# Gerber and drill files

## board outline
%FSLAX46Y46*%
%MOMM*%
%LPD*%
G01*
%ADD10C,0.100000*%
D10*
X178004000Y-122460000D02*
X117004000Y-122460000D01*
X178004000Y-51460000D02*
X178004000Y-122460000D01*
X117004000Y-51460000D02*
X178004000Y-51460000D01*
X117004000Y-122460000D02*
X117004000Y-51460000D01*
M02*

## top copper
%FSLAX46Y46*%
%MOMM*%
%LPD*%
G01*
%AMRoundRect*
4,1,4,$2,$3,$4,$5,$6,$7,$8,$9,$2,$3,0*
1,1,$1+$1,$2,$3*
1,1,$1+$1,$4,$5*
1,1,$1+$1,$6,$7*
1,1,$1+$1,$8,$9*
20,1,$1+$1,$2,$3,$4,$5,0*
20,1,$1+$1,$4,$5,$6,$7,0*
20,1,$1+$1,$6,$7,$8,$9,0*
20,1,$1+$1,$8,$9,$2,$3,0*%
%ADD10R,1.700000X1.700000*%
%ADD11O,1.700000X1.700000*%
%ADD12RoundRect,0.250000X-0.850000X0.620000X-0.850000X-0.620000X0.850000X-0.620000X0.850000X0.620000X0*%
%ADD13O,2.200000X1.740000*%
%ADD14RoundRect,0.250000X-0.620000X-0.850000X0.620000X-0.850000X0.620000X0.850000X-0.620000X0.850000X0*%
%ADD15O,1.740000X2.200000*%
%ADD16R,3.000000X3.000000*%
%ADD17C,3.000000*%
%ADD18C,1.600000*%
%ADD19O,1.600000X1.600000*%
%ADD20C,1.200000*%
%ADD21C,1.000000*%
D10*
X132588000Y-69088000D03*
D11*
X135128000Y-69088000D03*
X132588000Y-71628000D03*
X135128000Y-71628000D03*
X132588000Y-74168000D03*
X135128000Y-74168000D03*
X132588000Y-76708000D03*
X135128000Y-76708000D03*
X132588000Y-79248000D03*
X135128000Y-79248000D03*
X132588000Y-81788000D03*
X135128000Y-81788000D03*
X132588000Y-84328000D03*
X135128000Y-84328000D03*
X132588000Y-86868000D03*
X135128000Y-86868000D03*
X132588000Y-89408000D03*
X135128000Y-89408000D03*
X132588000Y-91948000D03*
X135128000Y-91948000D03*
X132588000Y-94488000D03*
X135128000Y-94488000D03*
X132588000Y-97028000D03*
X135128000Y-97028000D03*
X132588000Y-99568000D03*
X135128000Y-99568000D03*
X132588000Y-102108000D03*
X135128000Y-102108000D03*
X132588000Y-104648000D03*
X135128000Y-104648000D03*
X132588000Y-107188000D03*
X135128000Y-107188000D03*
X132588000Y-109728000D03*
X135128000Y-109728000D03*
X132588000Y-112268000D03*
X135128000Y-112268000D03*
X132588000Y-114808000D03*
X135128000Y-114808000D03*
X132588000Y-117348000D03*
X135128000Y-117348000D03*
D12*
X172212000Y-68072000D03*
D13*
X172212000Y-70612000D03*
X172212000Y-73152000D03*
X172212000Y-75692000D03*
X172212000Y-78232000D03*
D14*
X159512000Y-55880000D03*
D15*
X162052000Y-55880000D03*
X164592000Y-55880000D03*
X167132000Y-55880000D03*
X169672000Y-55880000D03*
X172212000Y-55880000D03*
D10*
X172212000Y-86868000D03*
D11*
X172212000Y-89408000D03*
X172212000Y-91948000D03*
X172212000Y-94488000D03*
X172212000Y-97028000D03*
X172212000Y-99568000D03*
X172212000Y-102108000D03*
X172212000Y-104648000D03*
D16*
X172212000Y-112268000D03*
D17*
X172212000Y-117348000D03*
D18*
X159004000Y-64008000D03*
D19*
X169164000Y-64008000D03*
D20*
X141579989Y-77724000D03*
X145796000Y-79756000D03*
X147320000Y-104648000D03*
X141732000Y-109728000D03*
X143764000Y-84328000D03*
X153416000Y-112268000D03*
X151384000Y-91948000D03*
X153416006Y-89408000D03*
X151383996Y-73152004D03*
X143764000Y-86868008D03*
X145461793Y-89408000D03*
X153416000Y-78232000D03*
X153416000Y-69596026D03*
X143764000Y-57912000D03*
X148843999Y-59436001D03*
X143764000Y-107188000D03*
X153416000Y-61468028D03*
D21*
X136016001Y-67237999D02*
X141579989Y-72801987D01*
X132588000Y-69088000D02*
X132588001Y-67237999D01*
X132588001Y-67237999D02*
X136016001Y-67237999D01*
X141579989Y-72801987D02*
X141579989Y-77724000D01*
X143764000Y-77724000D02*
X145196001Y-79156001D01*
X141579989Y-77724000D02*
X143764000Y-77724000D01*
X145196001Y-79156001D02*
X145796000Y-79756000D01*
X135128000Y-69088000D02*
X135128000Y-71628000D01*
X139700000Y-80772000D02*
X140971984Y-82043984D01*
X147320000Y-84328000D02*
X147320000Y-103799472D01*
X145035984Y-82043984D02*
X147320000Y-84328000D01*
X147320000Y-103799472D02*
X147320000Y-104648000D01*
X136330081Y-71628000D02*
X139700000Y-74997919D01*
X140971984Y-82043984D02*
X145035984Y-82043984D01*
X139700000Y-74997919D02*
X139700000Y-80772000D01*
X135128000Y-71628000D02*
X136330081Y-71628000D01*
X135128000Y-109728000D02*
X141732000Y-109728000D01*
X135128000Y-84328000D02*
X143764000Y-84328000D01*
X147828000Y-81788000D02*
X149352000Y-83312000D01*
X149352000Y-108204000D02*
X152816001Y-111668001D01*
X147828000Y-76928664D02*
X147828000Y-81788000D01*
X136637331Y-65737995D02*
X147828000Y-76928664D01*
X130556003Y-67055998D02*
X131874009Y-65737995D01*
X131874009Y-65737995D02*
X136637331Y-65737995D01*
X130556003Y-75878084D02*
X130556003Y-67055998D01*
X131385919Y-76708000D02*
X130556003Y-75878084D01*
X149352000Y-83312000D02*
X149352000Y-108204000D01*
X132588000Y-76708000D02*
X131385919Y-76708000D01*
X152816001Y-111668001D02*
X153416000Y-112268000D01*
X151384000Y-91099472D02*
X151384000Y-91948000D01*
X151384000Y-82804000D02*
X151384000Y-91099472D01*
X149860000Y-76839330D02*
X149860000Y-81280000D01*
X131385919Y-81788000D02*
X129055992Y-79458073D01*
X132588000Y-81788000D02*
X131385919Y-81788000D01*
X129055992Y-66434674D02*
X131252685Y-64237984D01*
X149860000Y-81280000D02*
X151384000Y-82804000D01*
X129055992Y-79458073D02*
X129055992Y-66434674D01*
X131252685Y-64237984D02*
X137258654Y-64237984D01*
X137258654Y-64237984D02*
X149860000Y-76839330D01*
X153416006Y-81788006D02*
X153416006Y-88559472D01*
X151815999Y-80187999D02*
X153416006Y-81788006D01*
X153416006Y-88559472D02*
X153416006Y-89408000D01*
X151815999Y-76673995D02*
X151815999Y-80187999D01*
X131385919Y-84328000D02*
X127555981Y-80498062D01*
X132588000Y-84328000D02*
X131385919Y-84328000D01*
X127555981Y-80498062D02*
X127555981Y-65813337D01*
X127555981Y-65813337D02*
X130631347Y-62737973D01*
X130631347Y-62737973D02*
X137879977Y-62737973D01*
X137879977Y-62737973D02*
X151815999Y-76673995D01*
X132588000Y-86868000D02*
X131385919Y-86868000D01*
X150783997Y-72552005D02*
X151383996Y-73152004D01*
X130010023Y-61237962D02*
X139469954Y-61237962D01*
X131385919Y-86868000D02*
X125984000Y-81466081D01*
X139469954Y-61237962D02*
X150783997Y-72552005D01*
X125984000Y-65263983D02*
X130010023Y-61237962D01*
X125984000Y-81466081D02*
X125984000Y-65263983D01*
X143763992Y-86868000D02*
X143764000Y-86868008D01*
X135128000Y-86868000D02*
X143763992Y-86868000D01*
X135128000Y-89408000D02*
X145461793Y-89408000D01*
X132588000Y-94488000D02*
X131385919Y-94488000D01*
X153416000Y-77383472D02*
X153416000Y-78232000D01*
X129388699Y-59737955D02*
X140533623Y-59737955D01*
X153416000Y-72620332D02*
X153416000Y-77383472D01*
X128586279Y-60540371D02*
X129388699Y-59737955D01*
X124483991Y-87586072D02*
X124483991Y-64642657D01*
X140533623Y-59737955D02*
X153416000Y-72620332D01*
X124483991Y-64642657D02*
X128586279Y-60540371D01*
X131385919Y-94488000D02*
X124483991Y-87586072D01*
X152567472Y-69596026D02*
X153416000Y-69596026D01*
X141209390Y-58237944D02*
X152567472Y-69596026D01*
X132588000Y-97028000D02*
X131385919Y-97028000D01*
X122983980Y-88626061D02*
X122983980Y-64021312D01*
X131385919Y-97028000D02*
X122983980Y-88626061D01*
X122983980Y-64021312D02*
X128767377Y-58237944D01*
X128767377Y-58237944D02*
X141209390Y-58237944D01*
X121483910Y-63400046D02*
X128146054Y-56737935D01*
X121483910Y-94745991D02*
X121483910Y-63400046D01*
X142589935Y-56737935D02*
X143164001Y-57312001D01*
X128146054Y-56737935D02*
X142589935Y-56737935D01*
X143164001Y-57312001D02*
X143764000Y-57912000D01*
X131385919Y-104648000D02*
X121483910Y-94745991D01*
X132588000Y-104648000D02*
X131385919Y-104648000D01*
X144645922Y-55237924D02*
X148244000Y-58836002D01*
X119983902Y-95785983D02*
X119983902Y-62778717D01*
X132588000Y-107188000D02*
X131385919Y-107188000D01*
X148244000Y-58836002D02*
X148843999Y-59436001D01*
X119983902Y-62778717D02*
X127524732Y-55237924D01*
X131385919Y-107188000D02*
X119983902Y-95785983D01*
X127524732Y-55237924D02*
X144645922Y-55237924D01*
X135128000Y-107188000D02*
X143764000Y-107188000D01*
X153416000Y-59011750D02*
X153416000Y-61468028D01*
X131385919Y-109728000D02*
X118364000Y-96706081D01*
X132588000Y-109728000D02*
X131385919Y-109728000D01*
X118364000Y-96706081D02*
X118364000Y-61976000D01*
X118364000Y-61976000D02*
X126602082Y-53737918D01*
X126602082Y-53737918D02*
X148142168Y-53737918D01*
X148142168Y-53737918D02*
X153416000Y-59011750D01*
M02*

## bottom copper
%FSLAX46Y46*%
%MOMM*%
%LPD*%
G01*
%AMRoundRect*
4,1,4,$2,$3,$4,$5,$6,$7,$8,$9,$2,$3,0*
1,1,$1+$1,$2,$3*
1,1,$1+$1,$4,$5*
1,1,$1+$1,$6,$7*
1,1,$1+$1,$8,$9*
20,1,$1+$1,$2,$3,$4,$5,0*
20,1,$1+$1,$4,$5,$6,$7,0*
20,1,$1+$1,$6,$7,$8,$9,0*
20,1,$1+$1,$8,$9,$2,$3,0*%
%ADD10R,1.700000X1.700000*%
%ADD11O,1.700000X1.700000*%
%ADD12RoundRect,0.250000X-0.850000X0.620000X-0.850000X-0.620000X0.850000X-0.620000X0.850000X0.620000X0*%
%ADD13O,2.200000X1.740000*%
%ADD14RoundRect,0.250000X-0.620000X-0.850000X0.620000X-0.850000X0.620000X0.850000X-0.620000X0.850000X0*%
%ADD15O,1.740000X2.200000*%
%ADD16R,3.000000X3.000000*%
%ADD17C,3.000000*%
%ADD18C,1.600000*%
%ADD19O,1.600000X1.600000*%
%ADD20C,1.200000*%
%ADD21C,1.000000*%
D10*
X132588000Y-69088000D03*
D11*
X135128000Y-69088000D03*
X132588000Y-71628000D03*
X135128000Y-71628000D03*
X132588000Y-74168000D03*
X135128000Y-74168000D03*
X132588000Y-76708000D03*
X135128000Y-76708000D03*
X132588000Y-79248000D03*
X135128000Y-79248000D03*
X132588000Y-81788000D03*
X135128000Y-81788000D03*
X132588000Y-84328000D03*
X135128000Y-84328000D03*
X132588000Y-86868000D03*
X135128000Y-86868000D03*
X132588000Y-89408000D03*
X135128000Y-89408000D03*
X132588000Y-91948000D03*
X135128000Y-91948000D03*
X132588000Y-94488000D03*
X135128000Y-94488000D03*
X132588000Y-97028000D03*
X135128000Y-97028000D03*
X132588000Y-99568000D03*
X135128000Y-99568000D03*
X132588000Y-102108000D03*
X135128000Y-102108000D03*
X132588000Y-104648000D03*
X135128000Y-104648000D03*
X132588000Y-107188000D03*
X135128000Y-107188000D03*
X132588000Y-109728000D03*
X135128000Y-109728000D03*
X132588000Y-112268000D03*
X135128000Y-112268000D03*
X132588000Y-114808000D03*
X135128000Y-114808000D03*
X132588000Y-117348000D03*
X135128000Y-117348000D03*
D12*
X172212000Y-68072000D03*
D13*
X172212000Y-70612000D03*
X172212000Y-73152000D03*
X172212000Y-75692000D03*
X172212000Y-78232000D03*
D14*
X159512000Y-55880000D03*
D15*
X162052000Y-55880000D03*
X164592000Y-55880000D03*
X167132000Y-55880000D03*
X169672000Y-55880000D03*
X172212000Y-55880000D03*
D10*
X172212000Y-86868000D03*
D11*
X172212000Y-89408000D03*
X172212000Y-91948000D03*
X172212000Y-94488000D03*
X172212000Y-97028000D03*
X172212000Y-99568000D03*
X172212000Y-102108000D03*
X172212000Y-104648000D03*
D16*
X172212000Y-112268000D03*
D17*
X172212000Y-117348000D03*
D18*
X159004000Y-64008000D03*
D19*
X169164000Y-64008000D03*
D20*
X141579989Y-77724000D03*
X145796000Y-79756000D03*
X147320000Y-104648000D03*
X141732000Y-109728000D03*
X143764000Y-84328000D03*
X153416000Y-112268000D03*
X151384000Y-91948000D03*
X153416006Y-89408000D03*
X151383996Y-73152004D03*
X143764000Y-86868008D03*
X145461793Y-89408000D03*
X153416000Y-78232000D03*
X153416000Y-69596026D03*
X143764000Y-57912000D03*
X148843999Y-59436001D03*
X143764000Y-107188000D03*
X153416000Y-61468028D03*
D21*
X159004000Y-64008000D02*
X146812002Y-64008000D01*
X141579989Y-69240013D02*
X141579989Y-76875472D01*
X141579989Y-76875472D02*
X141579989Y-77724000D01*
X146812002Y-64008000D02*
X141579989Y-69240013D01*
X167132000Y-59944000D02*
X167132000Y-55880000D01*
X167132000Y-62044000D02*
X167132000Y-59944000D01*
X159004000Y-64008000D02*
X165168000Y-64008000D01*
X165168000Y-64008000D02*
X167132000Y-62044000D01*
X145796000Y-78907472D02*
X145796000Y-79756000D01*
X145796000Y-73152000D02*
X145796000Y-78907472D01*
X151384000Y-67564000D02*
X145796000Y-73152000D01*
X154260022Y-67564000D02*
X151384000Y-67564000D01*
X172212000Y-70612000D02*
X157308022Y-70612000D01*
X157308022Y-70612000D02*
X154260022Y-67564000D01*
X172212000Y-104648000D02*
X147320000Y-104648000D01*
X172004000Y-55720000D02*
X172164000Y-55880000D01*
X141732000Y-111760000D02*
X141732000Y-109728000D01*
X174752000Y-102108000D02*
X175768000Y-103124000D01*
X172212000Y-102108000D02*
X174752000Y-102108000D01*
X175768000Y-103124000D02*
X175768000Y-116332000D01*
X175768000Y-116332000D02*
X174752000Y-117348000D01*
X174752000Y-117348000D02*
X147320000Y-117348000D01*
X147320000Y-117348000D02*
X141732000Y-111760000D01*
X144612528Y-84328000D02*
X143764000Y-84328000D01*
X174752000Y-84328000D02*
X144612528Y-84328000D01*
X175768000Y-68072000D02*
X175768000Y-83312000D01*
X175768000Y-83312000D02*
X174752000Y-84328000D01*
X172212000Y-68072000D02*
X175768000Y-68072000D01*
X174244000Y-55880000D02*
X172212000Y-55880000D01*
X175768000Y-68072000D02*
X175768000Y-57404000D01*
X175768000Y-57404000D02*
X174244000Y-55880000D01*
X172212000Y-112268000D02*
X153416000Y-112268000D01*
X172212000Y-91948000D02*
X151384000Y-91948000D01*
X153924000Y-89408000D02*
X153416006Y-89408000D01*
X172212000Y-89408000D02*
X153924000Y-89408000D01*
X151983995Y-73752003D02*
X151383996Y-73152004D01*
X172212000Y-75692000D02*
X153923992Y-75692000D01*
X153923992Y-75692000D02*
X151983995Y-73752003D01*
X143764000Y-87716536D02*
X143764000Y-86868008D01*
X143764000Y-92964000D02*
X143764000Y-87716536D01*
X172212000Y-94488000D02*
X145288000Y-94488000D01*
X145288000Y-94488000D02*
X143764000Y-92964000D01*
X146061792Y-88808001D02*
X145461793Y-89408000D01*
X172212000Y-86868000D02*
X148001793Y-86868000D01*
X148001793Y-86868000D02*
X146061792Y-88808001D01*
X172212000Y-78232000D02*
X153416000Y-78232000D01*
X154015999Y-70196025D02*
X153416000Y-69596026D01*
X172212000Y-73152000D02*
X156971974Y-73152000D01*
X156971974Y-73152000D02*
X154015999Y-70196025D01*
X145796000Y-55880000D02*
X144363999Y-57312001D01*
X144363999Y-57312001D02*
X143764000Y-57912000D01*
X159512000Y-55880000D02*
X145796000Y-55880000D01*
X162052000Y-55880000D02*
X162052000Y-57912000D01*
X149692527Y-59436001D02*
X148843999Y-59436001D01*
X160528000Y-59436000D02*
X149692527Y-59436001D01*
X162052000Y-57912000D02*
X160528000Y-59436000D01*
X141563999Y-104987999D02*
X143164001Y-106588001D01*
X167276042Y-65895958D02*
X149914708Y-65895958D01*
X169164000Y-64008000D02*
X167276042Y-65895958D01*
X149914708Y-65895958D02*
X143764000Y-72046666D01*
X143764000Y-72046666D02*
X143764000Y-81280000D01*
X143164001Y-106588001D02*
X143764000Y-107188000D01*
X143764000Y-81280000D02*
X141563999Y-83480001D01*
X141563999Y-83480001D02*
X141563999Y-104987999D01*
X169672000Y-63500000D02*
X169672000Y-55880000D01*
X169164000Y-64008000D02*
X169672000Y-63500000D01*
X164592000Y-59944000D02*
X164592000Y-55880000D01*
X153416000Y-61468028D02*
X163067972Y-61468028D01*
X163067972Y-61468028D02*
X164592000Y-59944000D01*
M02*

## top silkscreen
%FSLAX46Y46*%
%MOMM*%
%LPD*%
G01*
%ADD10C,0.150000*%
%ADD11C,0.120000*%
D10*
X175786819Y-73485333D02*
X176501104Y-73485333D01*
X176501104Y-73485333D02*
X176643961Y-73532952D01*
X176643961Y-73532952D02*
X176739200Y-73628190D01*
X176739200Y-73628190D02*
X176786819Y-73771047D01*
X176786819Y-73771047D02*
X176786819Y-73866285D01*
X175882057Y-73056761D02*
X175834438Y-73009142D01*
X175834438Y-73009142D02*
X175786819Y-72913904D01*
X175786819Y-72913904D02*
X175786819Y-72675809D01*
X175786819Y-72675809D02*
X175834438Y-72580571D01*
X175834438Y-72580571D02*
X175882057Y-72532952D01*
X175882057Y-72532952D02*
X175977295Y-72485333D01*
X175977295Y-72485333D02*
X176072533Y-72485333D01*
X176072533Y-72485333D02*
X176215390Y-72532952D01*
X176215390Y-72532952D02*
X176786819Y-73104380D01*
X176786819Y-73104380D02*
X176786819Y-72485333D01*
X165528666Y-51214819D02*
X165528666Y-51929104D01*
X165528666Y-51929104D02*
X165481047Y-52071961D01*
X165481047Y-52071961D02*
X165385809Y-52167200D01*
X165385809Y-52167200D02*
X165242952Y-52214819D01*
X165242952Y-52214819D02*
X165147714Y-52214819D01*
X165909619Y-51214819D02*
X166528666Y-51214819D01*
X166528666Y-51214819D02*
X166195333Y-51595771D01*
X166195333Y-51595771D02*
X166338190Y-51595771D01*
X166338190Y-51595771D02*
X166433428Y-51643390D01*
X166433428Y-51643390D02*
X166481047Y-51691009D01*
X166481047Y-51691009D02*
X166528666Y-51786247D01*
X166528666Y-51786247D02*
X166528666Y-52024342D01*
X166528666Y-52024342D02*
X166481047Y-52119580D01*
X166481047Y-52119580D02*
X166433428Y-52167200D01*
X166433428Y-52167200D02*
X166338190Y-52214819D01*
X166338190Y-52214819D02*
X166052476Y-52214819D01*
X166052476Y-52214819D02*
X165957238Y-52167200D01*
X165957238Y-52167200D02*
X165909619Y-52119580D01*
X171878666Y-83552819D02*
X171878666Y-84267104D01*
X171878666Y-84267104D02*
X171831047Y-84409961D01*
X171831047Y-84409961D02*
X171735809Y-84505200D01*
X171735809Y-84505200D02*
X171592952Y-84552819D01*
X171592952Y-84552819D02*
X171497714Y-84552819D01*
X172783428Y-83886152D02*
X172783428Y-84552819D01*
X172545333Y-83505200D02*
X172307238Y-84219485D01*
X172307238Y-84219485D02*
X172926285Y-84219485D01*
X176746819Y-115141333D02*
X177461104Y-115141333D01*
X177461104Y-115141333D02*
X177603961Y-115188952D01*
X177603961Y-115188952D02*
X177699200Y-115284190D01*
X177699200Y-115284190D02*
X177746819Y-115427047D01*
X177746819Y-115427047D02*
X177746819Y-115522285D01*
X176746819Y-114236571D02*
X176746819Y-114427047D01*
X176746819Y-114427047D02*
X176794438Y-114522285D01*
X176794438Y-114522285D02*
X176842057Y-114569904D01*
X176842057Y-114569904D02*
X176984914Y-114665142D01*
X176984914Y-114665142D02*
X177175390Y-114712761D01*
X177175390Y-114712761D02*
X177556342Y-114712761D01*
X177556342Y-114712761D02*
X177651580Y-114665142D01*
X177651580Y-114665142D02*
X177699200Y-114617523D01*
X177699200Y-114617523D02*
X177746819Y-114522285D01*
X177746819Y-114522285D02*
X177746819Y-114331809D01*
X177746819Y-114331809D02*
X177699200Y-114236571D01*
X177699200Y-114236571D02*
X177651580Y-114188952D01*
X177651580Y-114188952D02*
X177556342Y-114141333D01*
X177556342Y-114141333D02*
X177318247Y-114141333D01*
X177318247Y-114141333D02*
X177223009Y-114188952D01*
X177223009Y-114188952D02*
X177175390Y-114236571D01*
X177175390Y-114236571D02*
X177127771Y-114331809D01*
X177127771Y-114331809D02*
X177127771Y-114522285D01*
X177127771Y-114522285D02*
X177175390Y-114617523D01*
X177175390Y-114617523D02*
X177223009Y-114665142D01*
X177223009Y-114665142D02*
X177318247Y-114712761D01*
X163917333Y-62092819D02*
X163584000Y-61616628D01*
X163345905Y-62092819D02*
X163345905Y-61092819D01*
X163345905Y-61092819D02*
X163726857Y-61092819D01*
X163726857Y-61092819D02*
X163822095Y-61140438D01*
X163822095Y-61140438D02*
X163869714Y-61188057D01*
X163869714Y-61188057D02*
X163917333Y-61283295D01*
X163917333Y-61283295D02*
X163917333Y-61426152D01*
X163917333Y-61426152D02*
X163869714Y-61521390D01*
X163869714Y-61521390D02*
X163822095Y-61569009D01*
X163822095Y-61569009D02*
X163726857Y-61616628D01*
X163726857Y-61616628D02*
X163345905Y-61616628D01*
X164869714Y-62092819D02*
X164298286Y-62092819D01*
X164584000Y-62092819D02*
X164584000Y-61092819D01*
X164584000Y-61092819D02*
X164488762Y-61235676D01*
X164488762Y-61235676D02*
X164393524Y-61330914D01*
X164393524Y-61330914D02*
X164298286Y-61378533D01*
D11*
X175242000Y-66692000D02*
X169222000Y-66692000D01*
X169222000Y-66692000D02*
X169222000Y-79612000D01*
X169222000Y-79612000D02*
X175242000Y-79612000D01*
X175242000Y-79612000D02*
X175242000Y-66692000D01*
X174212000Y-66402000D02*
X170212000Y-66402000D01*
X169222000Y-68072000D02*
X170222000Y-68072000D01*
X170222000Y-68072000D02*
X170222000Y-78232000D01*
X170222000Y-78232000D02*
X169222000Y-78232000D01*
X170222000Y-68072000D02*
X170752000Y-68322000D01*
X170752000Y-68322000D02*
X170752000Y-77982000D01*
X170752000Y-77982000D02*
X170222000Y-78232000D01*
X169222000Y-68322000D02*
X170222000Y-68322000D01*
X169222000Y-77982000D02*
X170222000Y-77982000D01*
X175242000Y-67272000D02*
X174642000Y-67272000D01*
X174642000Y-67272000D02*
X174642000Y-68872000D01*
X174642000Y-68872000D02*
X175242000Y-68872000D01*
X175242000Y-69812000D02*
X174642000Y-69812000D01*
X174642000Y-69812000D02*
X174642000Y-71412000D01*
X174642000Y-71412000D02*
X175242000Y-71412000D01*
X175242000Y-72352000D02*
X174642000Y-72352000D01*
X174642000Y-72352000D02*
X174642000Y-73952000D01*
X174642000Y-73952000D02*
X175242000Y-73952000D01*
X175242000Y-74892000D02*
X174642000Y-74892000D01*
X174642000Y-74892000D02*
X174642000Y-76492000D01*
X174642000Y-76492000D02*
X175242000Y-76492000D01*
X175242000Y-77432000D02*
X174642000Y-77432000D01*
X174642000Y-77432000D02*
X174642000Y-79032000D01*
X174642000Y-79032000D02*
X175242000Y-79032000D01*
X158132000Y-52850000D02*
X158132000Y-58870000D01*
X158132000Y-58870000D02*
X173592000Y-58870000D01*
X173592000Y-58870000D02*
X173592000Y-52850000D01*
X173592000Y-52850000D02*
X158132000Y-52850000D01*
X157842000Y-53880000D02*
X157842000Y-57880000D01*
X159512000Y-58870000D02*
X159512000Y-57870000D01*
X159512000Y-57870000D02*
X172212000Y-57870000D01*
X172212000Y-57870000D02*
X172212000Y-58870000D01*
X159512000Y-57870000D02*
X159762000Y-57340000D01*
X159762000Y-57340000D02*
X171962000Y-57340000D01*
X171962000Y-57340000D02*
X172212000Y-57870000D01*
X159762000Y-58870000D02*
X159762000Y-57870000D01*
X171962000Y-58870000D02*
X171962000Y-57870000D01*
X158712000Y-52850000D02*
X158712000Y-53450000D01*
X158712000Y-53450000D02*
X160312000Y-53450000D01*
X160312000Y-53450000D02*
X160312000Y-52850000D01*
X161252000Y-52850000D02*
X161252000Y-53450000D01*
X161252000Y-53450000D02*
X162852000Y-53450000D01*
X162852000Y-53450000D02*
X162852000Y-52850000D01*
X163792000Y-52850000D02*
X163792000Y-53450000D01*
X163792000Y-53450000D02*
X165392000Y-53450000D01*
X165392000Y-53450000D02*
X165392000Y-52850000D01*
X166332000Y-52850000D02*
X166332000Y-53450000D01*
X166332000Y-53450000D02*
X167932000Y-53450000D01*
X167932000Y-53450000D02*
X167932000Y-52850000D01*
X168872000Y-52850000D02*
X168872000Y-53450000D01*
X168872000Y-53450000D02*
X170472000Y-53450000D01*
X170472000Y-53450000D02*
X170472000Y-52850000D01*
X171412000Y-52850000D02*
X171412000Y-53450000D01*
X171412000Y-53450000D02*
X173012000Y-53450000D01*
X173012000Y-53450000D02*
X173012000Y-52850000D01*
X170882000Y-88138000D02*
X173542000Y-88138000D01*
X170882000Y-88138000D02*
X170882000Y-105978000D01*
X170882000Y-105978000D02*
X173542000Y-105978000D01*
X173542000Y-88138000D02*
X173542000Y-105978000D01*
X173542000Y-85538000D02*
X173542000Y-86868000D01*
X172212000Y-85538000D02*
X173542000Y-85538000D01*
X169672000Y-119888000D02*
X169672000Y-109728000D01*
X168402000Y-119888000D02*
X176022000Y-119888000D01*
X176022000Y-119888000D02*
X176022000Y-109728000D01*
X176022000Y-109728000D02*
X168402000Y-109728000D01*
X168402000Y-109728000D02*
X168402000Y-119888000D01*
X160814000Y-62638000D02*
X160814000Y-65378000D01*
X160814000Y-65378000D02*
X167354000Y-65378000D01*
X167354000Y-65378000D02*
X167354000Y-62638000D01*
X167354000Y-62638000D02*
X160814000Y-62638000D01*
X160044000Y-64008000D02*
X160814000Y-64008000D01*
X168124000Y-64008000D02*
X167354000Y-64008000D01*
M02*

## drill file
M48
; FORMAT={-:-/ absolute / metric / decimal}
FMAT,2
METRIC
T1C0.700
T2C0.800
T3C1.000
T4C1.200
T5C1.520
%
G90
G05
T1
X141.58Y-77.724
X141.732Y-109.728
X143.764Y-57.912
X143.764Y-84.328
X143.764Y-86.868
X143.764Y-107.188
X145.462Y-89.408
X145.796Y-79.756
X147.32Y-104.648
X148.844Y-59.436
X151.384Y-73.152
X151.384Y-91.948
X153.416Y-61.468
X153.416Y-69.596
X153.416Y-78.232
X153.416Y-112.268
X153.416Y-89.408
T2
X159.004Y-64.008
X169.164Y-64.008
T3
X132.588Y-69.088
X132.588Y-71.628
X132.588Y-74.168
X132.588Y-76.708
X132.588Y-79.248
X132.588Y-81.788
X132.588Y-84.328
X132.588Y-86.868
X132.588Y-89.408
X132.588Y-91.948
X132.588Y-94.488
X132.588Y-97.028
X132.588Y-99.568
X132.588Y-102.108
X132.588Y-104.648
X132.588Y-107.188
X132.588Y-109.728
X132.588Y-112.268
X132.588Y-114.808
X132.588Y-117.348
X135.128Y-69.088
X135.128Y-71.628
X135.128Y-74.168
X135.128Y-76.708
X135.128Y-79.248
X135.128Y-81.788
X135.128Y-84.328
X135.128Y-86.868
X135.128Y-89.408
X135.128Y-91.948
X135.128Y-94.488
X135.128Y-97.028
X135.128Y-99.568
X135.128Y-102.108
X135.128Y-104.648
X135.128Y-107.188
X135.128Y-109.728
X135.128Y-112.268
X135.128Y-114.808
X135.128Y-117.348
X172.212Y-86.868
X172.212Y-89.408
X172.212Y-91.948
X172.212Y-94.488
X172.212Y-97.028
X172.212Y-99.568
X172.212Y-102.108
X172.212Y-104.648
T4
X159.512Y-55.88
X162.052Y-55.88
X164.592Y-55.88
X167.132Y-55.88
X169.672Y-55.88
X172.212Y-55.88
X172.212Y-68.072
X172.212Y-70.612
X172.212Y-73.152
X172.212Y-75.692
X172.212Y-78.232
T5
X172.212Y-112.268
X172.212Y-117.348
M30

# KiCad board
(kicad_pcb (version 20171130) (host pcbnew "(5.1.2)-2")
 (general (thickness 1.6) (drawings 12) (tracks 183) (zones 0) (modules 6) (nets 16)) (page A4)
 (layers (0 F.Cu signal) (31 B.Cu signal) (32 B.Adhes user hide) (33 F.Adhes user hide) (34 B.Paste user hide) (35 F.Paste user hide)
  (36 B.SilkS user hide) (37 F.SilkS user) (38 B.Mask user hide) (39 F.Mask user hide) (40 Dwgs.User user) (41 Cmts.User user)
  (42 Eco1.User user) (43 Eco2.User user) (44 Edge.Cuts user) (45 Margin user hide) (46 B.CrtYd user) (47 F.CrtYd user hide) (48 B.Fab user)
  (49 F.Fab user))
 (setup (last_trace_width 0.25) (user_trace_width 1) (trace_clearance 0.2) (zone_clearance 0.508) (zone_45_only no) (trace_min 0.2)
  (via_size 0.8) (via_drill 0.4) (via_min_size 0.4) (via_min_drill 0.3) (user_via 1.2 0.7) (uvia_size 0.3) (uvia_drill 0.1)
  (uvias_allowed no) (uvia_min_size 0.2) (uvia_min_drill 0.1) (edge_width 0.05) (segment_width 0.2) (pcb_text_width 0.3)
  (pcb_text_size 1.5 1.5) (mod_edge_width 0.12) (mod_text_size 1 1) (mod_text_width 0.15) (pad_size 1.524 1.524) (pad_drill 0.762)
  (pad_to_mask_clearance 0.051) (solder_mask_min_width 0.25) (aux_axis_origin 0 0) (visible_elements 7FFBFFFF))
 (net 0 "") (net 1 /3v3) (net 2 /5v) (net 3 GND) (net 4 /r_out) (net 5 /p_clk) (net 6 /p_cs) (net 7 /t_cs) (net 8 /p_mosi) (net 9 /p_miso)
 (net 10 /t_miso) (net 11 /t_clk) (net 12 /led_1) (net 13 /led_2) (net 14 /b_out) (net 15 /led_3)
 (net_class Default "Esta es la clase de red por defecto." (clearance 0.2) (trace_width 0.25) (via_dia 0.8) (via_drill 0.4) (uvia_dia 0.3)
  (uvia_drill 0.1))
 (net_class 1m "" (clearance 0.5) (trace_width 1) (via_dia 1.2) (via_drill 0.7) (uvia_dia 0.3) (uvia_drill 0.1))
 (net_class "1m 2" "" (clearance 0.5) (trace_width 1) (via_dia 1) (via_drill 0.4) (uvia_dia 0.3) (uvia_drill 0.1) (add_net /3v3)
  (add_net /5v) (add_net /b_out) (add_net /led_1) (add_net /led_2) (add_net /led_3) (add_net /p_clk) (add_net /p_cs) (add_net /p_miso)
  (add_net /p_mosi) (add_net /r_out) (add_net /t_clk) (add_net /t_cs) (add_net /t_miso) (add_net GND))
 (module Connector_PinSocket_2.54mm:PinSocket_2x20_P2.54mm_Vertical (layer B.Cu) (at 132.588 69.088 180)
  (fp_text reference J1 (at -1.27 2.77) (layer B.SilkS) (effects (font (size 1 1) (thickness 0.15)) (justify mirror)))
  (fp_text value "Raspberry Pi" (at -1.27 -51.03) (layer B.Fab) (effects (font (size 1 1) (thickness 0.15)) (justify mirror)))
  (pad 1 thru_hole rect (at 0 0 180) (size 1.7 1.7) (drill 1) (layers *.Cu *.Mask) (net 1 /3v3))
  (pad 2 thru_hole oval (at -2.54 0 180) (size 1.7 1.7) (drill 1) (layers *.Cu *.Mask) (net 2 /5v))
  (pad 3 thru_hole oval (at 0 -2.54 180) (size 1.7 1.7) (drill 1) (layers *.Cu *.Mask))
  (pad 4 thru_hole oval (at -2.54 -2.54 180) (size 1.7 1.7) (drill 1) (layers *.Cu *.Mask) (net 2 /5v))
  (pad 5 thru_hole oval (at 0 -5.08 180) (size 1.7 1.7) (drill 1) (layers *.Cu *.Mask))
  (pad 6 thru_hole oval (at -2.54 -5.08 180) (size 1.7 1.7) (drill 1) (layers *.Cu *.Mask) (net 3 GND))
  (pad 7 thru_hole oval (at 0 -7.62 180) (size 1.7 1.7) (drill 1) (layers *.Cu *.Mask) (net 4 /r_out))
  (pad 8 thru_hole oval (at -2.54 -7.62 180) (size 1.7 1.7) (drill 1) (layers *.Cu *.Mask))
  (pad 9 thru_hole oval (at 0 -10.16 180) (size 1.7 1.7) (drill 1) (layers *.Cu *.Mask))
  (pad 10 thru_hole oval (at -2.54 -10.16 180) (size 1.7 1.7) (drill 1) (layers *.Cu *.Mask))
  (pad 11 thru_hole oval (at 0 -12.7 180) (size 1.7 1.7) (drill 1) (layers *.Cu *.Mask) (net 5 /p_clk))
  (pad 12 thru_hole oval (at -2.54 -12.7 180) (size 1.7 1.7) (drill 1) (layers *.Cu *.Mask))
  (pad 13 thru_hole oval (at 0 -15.24 180) (size 1.7 1.7) (drill 1) (layers *.Cu *.Mask) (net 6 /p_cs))
  (pad 14 thru_hole oval (at -2.54 -15.24 180) (size 1.7 1.7) (drill 1) (layers *.Cu *.Mask) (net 3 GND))
  (pad 15 thru_hole oval (at 0 -17.78 180) (size 1.7 1.7) (drill 1) (layers *.Cu *.Mask) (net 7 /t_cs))
  (pad 16 thru_hole oval (at -2.54 -17.78 180) (size 1.7 1.7) (drill 1) (layers *.Cu *.Mask) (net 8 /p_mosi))
  (pad 17 thru_hole oval (at 0 -20.32 180) (size 1.7 1.7) (drill 1) (layers *.Cu *.Mask))
  (pad 18 thru_hole oval (at -2.54 -20.32 180) (size 1.7 1.7) (drill 1) (layers *.Cu *.Mask) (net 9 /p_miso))
  (pad 19 thru_hole oval (at 0 -22.86 180) (size 1.7 1.7) (drill 1) (layers *.Cu *.Mask))
  (pad 20 thru_hole oval (at -2.54 -22.86 180) (size 1.7 1.7) (drill 1) (layers *.Cu *.Mask) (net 3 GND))
  (pad 21 thru_hole oval (at 0 -25.4 180) (size 1.7 1.7) (drill 1) (layers *.Cu *.Mask) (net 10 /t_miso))
  (pad 22 thru_hole oval (at -2.54 -25.4 180) (size 1.7 1.7) (drill 1) (layers *.Cu *.Mask))
  (pad 23 thru_hole oval (at 0 -27.94 180) (size 1.7 1.7) (drill 1) (layers *.Cu *.Mask) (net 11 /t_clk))
  (pad 24 thru_hole oval (at -2.54 -27.94 180) (size 1.7 1.7) (drill 1) (layers *.Cu *.Mask))
  (pad 25 thru_hole oval (at 0 -30.48 180) (size 1.7 1.7) (drill 1) (layers *.Cu *.Mask))
  (pad 26 thru_hole oval (at -2.54 -30.48 180) (size 1.7 1.7) (drill 1) (layers *.Cu *.Mask))
  (pad 27 thru_hole oval (at 0 -33.02 180) (size 1.7 1.7) (drill 1) (layers *.Cu *.Mask))
  (pad 28 thru_hole oval (at -2.54 -33.02 180) (size 1.7 1.7) (drill 1) (layers *.Cu *.Mask))
  (pad 29 thru_hole oval (at 0 -35.56 180) (size 1.7 1.7) (drill 1) (layers *.Cu *.Mask) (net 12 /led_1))
  (pad 30 thru_hole oval (at -2.54 -35.56 180) (size 1.7 1.7) (drill 1) (layers *.Cu *.Mask) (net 3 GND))
  (pad 31 thru_hole oval (at 0 -38.1 180) (size 1.7 1.7) (drill 1) (layers *.Cu *.Mask) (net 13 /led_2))
  (pad 32 thru_hole oval (at -2.54 -38.1 180) (size 1.7 1.7) (drill 1) (layers *.Cu *.Mask) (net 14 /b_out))
  (pad 33 thru_hole oval (at 0 -40.64 180) (size 1.7 1.7) (drill 1) (layers *.Cu *.Mask) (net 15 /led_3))
  (pad 34 thru_hole oval (at -2.54 -40.64 180) (size 1.7 1.7) (drill 1) (layers *.Cu *.Mask) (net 3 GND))
  (pad 35 thru_hole oval (at 0 -43.18 180) (size 1.7 1.7) (drill 1) (layers *.Cu *.Mask))
  (pad 36 thru_hole oval (at -2.54 -43.18 180) (size 1.7 1.7) (drill 1) (layers *.Cu *.Mask))
  (pad 37 thru_hole oval (at 0 -45.72 180) (size 1.7 1.7) (drill 1) (layers *.Cu *.Mask))
  (pad 38 thru_hole oval (at -2.54 -45.72 180) (size 1.7 1.7) (drill 1) (layers *.Cu *.Mask))
  (pad 39 thru_hole oval (at 0 -48.26 180) (size 1.7 1.7) (drill 1) (layers *.Cu *.Mask))
  (pad 40 thru_hole oval (at -2.54 -48.26 180) (size 1.7 1.7) (drill 1) (layers *.Cu *.Mask)))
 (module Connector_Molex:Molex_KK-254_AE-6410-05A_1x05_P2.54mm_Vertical (layer F.Cu) (at 172.212 68.072 270)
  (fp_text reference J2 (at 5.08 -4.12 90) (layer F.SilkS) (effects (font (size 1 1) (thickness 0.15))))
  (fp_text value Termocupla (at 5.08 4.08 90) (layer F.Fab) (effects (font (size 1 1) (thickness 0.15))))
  (fp_line (start -1.38 -3.03) (end -1.38 2.99) (layer F.SilkS) (width 0.12))
  (fp_line (start -1.38 2.99) (end 11.54 2.99) (layer F.SilkS) (width 0.12))
  (fp_line (start 11.54 2.99) (end 11.54 -3.03) (layer F.SilkS) (width 0.12))
  (fp_line (start 11.54 -3.03) (end -1.38 -3.03) (layer F.SilkS) (width 0.12))
  (fp_line (start -1.67 -2) (end -1.67 2) (layer F.SilkS) (width 0.12))
  (fp_line (start 0 2.99) (end 0 1.99) (layer F.SilkS) (width 0.12))
  (fp_line (start 0 1.99) (end 10.16 1.99) (layer F.SilkS) (width 0.12))
  (fp_line (start 10.16 1.99) (end 10.16 2.99) (layer F.SilkS) (width 0.12))
  (fp_line (start 0 1.99) (end 0.25 1.46) (layer F.SilkS) (width 0.12))
  (fp_line (start 0.25 1.46) (end 9.91 1.46) (layer F.SilkS) (width 0.12))
  (fp_line (start 9.91 1.46) (end 10.16 1.99) (layer F.SilkS) (width 0.12))
  (fp_line (start 0.25 2.99) (end 0.25 1.99) (layer F.SilkS) (width 0.12))
  (fp_line (start 9.91 2.99) (end 9.91 1.99) (layer F.SilkS) (width 0.12))
  (fp_line (start -0.8 -3.03) (end -0.8 -2.43) (layer F.SilkS) (width 0.12))
  (fp_line (start -0.8 -2.43) (end 0.8 -2.43) (layer F.SilkS) (width 0.12))
  (fp_line (start 0.8 -2.43) (end 0.8 -3.03) (layer F.SilkS) (width 0.12))
  (fp_line (start 1.74 -3.03) (end 1.74 -2.43) (layer F.SilkS) (width 0.12))
  (fp_line (start 1.74 -2.43) (end 3.34 -2.43) (layer F.SilkS) (width 0.12))
  (fp_line (start 3.34 -2.43) (end 3.34 -3.03) (layer F.SilkS) (width 0.12))
  (fp_line (start 4.28 -3.03) (end 4.28 -2.43) (layer F.SilkS) (width 0.12))
  (fp_line (start 4.28 -2.43) (end 5.88 -2.43) (layer F.SilkS) (width 0.12))
  (fp_line (start 5.88 -2.43) (end 5.88 -3.03) (layer F.SilkS) (width 0.12))
  (fp_line (start 6.82 -3.03) (end 6.82 -2.43) (layer F.SilkS) (width 0.12))
  (fp_line (start 6.82 -2.43) (end 8.42 -2.43) (layer F.SilkS) (width 0.12))
  (fp_line (start 8.42 -2.43) (end 8.42 -3.03) (layer F.SilkS) (width 0.12))
  (fp_line (start 9.36 -3.03) (end 9.36 -2.43) (layer F.SilkS) (width 0.12))
  (fp_line (start 9.36 -2.43) (end 10.96 -2.43) (layer F.SilkS) (width 0.12))
  (fp_line (start 10.96 -2.43) (end 10.96 -3.03) (layer F.SilkS) (width 0.12))
  (pad 1 thru_hole roundrect (at 0 0 270) (size 1.74 2.2) (drill 1.2) (layers *.Cu *.Mask) (roundrect_rratio 0.143678) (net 3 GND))
  (pad 2 thru_hole oval (at 2.54 0 270) (size 1.74 2.2) (drill 1.2) (layers *.Cu *.Mask) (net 1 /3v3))
  (pad 3 thru_hole oval (at 5.08 0 270) (size 1.74 2.2) (drill 1.2) (layers *.Cu *.Mask) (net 11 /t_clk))
  (pad 4 thru_hole oval (at 7.62 0 270) (size 1.74 2.2) (drill 1.2) (layers *.Cu *.Mask) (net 7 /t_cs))
  (pad 5 thru_hole oval (at 10.16 0 270) (size 1.74 2.2) (drill 1.2) (layers *.Cu *.Mask) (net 10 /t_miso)))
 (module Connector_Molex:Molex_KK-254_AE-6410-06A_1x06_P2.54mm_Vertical (layer F.Cu) (at 159.512 55.88)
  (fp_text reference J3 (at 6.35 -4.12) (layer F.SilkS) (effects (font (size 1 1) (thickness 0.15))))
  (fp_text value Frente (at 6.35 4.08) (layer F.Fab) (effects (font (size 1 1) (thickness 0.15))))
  (fp_line (start -1.38 -3.03) (end -1.38 2.99) (layer F.SilkS) (width 0.12))
  (fp_line (start -1.38 2.99) (end 14.08 2.99) (layer F.SilkS) (width 0.12))
  (fp_line (start 14.08 2.99) (end 14.08 -3.03) (layer F.SilkS) (width 0.12))
  (fp_line (start 14.08 -3.03) (end -1.38 -3.03) (layer F.SilkS) (width 0.12))
  (fp_line (start -1.67 -2) (end -1.67 2) (layer F.SilkS) (width 0.12))
  (fp_line (start 0 2.99) (end 0 1.99) (layer F.SilkS) (width 0.12))
  (fp_line (start 0 1.99) (end 12.7 1.99) (layer F.SilkS) (width 0.12))
  (fp_line (start 12.7 1.99) (end 12.7 2.99) (layer F.SilkS) (width 0.12))
  (fp_line (start 0 1.99) (end 0.25 1.46) (layer F.SilkS) (width 0.12))
  (fp_line (start 0.25 1.46) (end 12.45 1.46) (layer F.SilkS) (width 0.12))
  (fp_line (start 12.45 1.46) (end 12.7 1.99) (layer F.SilkS) (width 0.12))
  (fp_line (start 0.25 2.99) (end 0.25 1.99) (layer F.SilkS) (width 0.12))
  (fp_line (start 12.45 2.99) (end 12.45 1.99) (layer F.SilkS) (width 0.12))
  (fp_line (start -0.8 -3.03) (end -0.8 -2.43) (layer F.SilkS) (width 0.12))
  (fp_line (start -0.8 -2.43) (end 0.8 -2.43) (layer F.SilkS) (width 0.12))
  (fp_line (start 0.8 -2.43) (end 0.8 -3.03) (layer F.SilkS) (width 0.12))
  (fp_line (start 1.74 -3.03) (end 1.74 -2.43) (layer F.SilkS) (width 0.12))
  (fp_line (start 1.74 -2.43) (end 3.34 -2.43) (layer F.SilkS) (width 0.12))
  (fp_line (start 3.34 -2.43) (end 3.34 -3.03) (layer F.SilkS) (width 0.12))
  (fp_line (start 4.28 -3.03) (end 4.28 -2.43) (layer F.SilkS) (width 0.12))
  (fp_line (start 4.28 -2.43) (end 5.88 -2.43) (layer F.SilkS) (width 0.12))
  (fp_line (start 5.88 -2.43) (end 5.88 -3.03) (layer F.SilkS) (width 0.12))
  (fp_line (start 6.82 -3.03) (end 6.82 -2.43) (layer F.SilkS) (width 0.12))
  (fp_line (start 6.82 -2.43) (end 8.42 -2.43) (layer F.SilkS) (width 0.12))
  (fp_line (start 8.42 -2.43) (end 8.42 -3.03) (layer F.SilkS) (width 0.12))
  (fp_line (start 9.36 -3.03) (end 9.36 -2.43) (layer F.SilkS) (width 0.12))
  (fp_line (start 9.36 -2.43) (end 10.96 -2.43) (layer F.SilkS) (width 0.12))
  (fp_line (start 10.96 -2.43) (end 10.96 -3.03) (layer F.SilkS) (width 0.12))
  (fp_line (start 11.9 -3.03) (end 11.9 -2.43) (layer F.SilkS) (width 0.12))
  (fp_line (start 11.9 -2.43) (end 13.5 -2.43) (layer F.SilkS) (width 0.12))
  (fp_line (start 13.5 -2.43) (end 13.5 -3.03) (layer F.SilkS) (width 0.12))
  (pad 1 thru_hole roundrect (at 0 0) (size 1.74 2.2) (drill 1.2) (layers *.Cu *.Mask) (roundrect_rratio 0.143678) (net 12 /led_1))
  (pad 2 thru_hole oval (at 2.54 0) (size 1.74 2.2) (drill 1.2) (layers *.Cu *.Mask) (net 13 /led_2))
  (pad 3 thru_hole oval (at 5.08 0) (size 1.74 2.2) (drill 1.2) (layers *.Cu *.Mask) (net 15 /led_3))
  (pad 4 thru_hole oval (at 7.62 0) (size 1.74 2.2) (drill 1.2) (layers *.Cu *.Mask) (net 1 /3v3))
  (pad 5 thru_hole oval (at 10.16 0) (size 1.74 2.2) (drill 1.2) (layers *.Cu *.Mask) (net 14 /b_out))
  (pad 6 thru_hole oval (at 12.7 0) (size 1.74 2.2) (drill 1.2) (layers *.Cu *.Mask) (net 3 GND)))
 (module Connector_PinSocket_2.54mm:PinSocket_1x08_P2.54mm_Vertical (layer F.Cu) (at 172.212 86.868)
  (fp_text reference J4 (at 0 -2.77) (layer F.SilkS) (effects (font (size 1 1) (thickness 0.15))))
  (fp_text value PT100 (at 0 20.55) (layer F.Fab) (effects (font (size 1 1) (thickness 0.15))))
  (fp_line (start -1.33 1.27) (end 1.33 1.27) (layer F.SilkS) (width 0.12))
  (fp_line (start -1.33 1.27) (end -1.33 19.11) (layer F.SilkS) (width 0.12))
  (fp_line (start -1.33 19.11) (end 1.33 19.11) (layer F.SilkS) (width 0.12))
  (fp_line (start 1.33 1.27) (end 1.33 19.11) (layer F.SilkS) (width 0.12))
  (fp_line (start 1.33 -1.33) (end 1.33 0) (layer F.SilkS) (width 0.12))
  (fp_line (start 0 -1.33) (end 1.33 -1.33) (layer F.SilkS) (width 0.12))
  (pad 1 thru_hole rect (at 0 0) (size 1.7 1.7) (drill 1) (layers *.Cu *.Mask) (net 9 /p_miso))
  (pad 2 thru_hole oval (at 0 2.54) (size 1.7 1.7) (drill 1) (layers *.Cu *.Mask) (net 6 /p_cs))
  (pad 3 thru_hole oval (at 0 5.08) (size 1.7 1.7) (drill 1) (layers *.Cu *.Mask) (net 5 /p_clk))
  (pad 4 thru_hole oval (at 0 7.62) (size 1.7 1.7) (drill 1) (layers *.Cu *.Mask) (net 8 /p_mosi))
  (pad 5 thru_hole oval (at 0 10.16) (size 1.7 1.7) (drill 1) (layers *.Cu *.Mask))
  (pad 6 thru_hole oval (at 0 12.7) (size 1.7 1.7) (drill 1) (layers *.Cu *.Mask))
  (pad 7 thru_hole oval (at 0 15.24) (size 1.7 1.7) (drill 1) (layers *.Cu *.Mask) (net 3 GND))
  (pad 8 thru_hole oval (at 0 17.78) (size 1.7 1.7) (drill 1) (layers *.Cu *.Mask) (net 2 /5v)))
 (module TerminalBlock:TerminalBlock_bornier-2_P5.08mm (layer F.Cu) (at 172.212 112.268 270)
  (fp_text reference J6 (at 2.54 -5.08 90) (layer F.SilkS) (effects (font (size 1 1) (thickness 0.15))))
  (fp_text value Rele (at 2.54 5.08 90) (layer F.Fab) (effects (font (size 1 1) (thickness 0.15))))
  (fp_line (start 7.62 2.54) (end -2.54 2.54) (layer F.SilkS) (width 0.12))
  (fp_line (start 7.62 3.81) (end 7.62 -3.81) (layer F.SilkS) (width 0.12))
  (fp_line (start 7.62 -3.81) (end -2.54 -3.81) (layer F.SilkS) (width 0.12))
  (fp_line (start -2.54 -3.81) (end -2.54 3.81) (layer F.SilkS) (width 0.12))
  (fp_line (start -2.54 3.81) (end 7.62 3.81) (layer F.SilkS) (width 0.12))
  (pad 1 thru_hole rect (at 0 0 270) (size 3 3) (drill 1.52) (layers *.Cu *.Mask) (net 4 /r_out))
  (pad 2 thru_hole circle (at 5.08 0 270) (size 3 3) (drill 1.52) (layers *.Cu *.Mask) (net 3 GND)))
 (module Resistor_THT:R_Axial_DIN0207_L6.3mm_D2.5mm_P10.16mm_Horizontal (layer F.Cu) (at 159.004 64.008)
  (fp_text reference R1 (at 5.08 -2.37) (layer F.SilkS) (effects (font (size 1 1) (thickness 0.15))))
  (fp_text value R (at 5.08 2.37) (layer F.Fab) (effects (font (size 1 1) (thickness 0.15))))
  (fp_line (start 1.81 -1.37) (end 1.81 1.37) (layer F.SilkS) (width 0.12))
  (fp_line (start 1.81 1.37) (end 8.35 1.37) (layer F.SilkS) (width 0.12))
  (fp_line (start 8.35 1.37) (end 8.35 -1.37) (layer F.SilkS) (width 0.12))
  (fp_line (start 8.35 -1.37) (end 1.81 -1.37) (layer F.SilkS) (width 0.12))
  (fp_line (start 1.04 0) (end 1.81 0) (layer F.SilkS) (width 0.12))
  (fp_line (start 9.12 0) (end 8.35 0) (layer F.SilkS) (width 0.12))
  (pad 1 thru_hole circle (at 0 0) (size 1.6 1.6) (drill 0.8) (layers *.Cu *.Mask) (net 1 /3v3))
  (pad 2 thru_hole oval (at 10.16 0) (size 1.6 1.6) (drill 0.8) (layers *.Cu *.Mask) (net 14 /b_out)))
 (gr_line (start 178.004 122.46) (end 117.004 122.46) (layer Edge.Cuts) (width 0.1))
 (gr_line (start 178.004 51.46) (end 178.004 122.46) (layer Edge.Cuts) (width 0.1))
 (gr_line (start 117.004 51.46) (end 178.004 51.46) (layer Edge.Cuts) (width 0.1))
 (gr_line (start 117.004 122.46) (end 117.004 51.46) (layer Edge.Cuts) (width 0.1))
 (segment (start 136.016001 67.237999) (end 141.579989 72.801987) (width 1) (layer F.Cu) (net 1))
 (segment (start 159.004 64.008) (end 146.812002 64.008) (width 1) (layer B.Cu) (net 1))
 (segment (start 141.579989 69.240013) (end 141.579989 76.875472) (width 1) (layer B.Cu) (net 1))
 (segment (start 141.579989 76.875472) (end 141.579989 77.724) (width 1) (layer B.Cu) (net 1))
 (segment (start 132.588 69.088) (end 132.588001 67.237999) (width 1) (layer F.Cu) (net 1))
 (segment (start 132.588001 67.237999) (end 136.016001 67.237999) (width 1) (layer F.Cu) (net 1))
 (segment (start 141.579989 72.801987) (end 141.579989 77.724) (width 1) (layer F.Cu) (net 1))
 (segment (start 146.812002 64.008) (end 141.579989 69.240013) (width 1) (layer B.Cu) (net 1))
 (via (at 141.579989 77.724) (size 1.2) (drill 0.7) (layers F.Cu B.Cu) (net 1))
 (via (at 145.796 79.756) (size 1.2) (drill 0.7) (layers F.Cu B.Cu) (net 1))
 (segment (start 143.764 77.724) (end 145.196001 79.156001) (width 1) (layer F.Cu) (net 1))
 (segment (start 141.579989 77.724) (end 143.764 77.724) (width 1) (layer F.Cu) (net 1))
 (segment (start 145.196001 79.156001) (end 145.796 79.756) (width 1) (layer F.Cu) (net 1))
 (segment (start 167.132 59.944) (end 167.132 55.88) (width 1) (layer B.Cu) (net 1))
 (segment (start 167.132 62.044) (end 167.132 59.944) (width 1) (layer B.Cu) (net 1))
 (segment (start 159.004 64.008) (end 165.168 64.008) (width 1) (layer B.Cu) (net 1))
 (segment (start 165.168 64.008) (end 167.132 62.044) (width 1) (layer B.Cu) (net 1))
 (segment (start 145.796 78.907472) (end 145.796 79.756) (width 1) (layer B.Cu) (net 1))
 (segment (start 145.796 73.152) (end 145.796 78.907472) (width 1) (layer B.Cu) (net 1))
 (segment (start 151.384 67.564) (end 145.796 73.152) (width 1) (layer B.Cu) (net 1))
 (segment (start 154.260022 67.564) (end 151.384 67.564) (width 1) (layer B.Cu) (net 1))
 (segment (start 172.212 70.612) (end 157.308022 70.612) (width 1) (layer B.Cu) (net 1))
 (segment (start 157.308022 70.612) (end 154.260022 67.564) (width 1) (layer B.Cu) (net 1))
 (segment (start 135.128 69.088) (end 135.128 71.628) (width 1) (layer F.Cu) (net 2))
 (via (at 147.32 104.648) (size 1.2) (drill 0.7) (layers F.Cu B.Cu) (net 2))
 (segment (start 139.7 80.772) (end 140.971984 82.043984) (width 1) (layer F.Cu) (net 2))
 (segment (start 147.32 84.328) (end 147.32 103.799472) (width 1) (layer F.Cu) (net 2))
 (segment (start 172.212 104.648) (end 147.32 104.648) (width 1) (layer B.Cu) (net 2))
 (segment (start 145.035984 82.043984) (end 147.32 84.328) (width 1) (layer F.Cu) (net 2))
 (segment (start 147.32 103.799472) (end 147.32 104.648) (width 1) (layer F.Cu) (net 2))
 (segment (start 136.330081 71.628) (end 139.7 74.997919) (width 1) (layer F.Cu) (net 2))
 (segment (start 140.971984 82.043984) (end 145.035984 82.043984) (width 1) (layer F.Cu) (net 2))
 (segment (start 139.7 74.997919) (end 139.7 80.772) (width 1) (layer F.Cu) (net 2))
 (segment (start 135.128 71.628) (end 136.330081 71.628) (width 1) (layer F.Cu) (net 2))
 (via (at 141.732 109.728) (size 1.2) (drill 0.7) (layers F.Cu B.Cu) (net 3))
 (segment (start 135.128 109.728) (end 141.732 109.728) (width 1) (layer F.Cu) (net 3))
 (via (at 143.764 84.328) (size 1.2) (drill 0.7) (layers F.Cu B.Cu) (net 3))
 (segment (start 135.128 84.328) (end 143.764 84.328) (width 1) (layer F.Cu) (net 3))
 (segment (start 172.004 55.72) (end 172.164 55.88) (width 1) (layer B.Cu) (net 3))
 (segment (start 141.732 111.76) (end 141.732 109.728) (width 1) (layer B.Cu) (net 3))
 (segment (start 174.752 102.108) (end 175.768 103.124) (width 1) (layer B.Cu) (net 3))
 (segment (start 172.212 102.108) (end 174.752 102.108) (width 1) (layer B.Cu) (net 3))
 (segment (start 175.768 103.124) (end 175.768 116.332) (width 1) (layer B.Cu) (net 3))
 (segment (start 175.768 116.332) (end 174.752 117.348) (width 1) (layer B.Cu) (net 3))
 (segment (start 174.752 117.348) (end 147.32 117.348) (width 1) (layer B.Cu) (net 3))
 (segment (start 147.32 117.348) (end 141.732 111.76) (width 1) (layer B.Cu) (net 3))
 (segment (start 144.612528 84.328) (end 143.764 84.328) (width 1) (layer B.Cu) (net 3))
 (segment (start 174.752 84.328) (end 144.612528 84.328) (width 1) (layer B.Cu) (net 3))
 (segment (start 175.768 68.072) (end 175.768 83.312) (width 1) (layer B.Cu) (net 3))
 (segment (start 175.768 83.312) (end 174.752 84.328) (width 1) (layer B.Cu) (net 3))
 (segment (start 172.212 68.072) (end 175.768 68.072) (width 1) (layer B.Cu) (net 3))
 (segment (start 174.244 55.88) (end 172.212 55.88) (width 1) (layer B.Cu) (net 3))
 (segment (start 175.768 68.072) (end 175.768 57.404) (width 1) (layer B.Cu) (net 3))
 (segment (start 175.768 57.404) (end 174.244 55.88) (width 1) (layer B.Cu) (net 3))
 (segment (start 147.828 81.788) (end 149.352 83.312) (width 1) (layer F.Cu) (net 4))
 (segment (start 149.352 108.204) (end 152.816001 111.668001) (width 1) (layer F.Cu) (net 4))
 (segment (start 147.828 76.928664) (end 147.828 81.788) (width 1) (layer F.Cu) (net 4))
 (segment (start 136.637331 65.737995) (end 147.828 76.928664) (width 1) (layer F.Cu) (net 4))
 (segment (start 130.556003 67.055998) (end 131.874009 65.737995) (width 1) (layer F.Cu) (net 4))
 (segment (start 131.874009 65.737995) (end 136.637331 65.737995) (width 1) (layer F.Cu) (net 4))
 (segment (start 130.556003 75.878084) (end 130.556003 67.055998) (width 1) (layer F.Cu) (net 4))
 (segment (start 131.385919 76.708) (end 130.556003 75.878084) (width 1) (layer F.Cu) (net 4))
 (segment (start 149.352 83.312) (end 149.352 108.204) (width 1) (layer F.Cu) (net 4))
 (segment (start 132.588 76.708) (end 131.385919 76.708) (width 1) (layer F.Cu) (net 4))
 (via (at 153.416 112.268) (size 1.2) (drill 0.7) (layers F.Cu B.Cu) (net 4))
 (segment (start 152.816001 111.668001) (end 153.416 112.268) (width 1) (layer F.Cu) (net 4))
 (segment (start 172.212 112.268) (end 153.416 112.268) (width 1) (layer B.Cu) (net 4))
 (via (at 151.384 91.948) (size 1.2) (drill 0.7) (layers F.Cu B.Cu) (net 5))
 (segment (start 151.384 91.099472) (end 151.384 91.948) (width 1) (layer F.Cu) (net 5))
 (segment (start 151.384 82.804) (end 151.384 91.099472) (width 1) (layer F.Cu) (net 5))
 (segment (start 149.86 76.83933) (end 149.86 81.28) (width 1) (layer F.Cu) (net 5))
 (segment (start 131.385919 81.788) (end 129.055992 79.458073) (width 1) (layer F.Cu) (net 5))
 (segment (start 132.588 81.788) (end 131.385919 81.788) (width 1) (layer F.Cu) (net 5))
 (segment (start 129.055992 66.434674) (end 131.252685 64.237984) (width 1) (layer F.Cu) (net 5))
 (segment (start 149.86 81.28) (end 151.384 82.804) (width 1) (layer F.Cu) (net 5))
 (segment (start 129.055992 79.458073) (end 129.055992 66.434674) (width 1) (layer F.Cu) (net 5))
 (segment (start 131.252685 64.237984) (end 137.258654 64.237984) (width 1) (layer F.Cu) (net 5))
 (segment (start 137.258654 64.237984) (end 149.86 76.83933) (width 1) (layer F.Cu) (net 5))
 (segment (start 172.212 91.948) (end 151.384 91.948) (width 1) (layer B.Cu) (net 5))
 (via (at 153.416006 89.408) (size 1.2) (drill 0.7) (layers F.Cu B.Cu) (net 6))
 (segment (start 153.416006 81.788006) (end 153.416006 88.559472) (width 1) (layer F.Cu) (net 6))
 (segment (start 151.815999 80.187999) (end 153.416006 81.788006) (width 1) (layer F.Cu) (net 6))
 (segment (start 153.416006 88.559472) (end 153.416006 89.408) (width 1) (layer F.Cu) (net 6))
 (segment (start 151.815999 76.673995) (end 151.815999 80.187999) (width 1) (layer F.Cu) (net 6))
 (segment (start 131.385919 84.328) (end 127.555981 80.498062) (width 1) (layer F.Cu) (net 6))
 (segment (start 132.588 84.328) (end 131.385919 84.328) (width 1) (layer F.Cu) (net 6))
 (segment (start 127.555981 80.498062) (end 127.555981 65.813337) (width 1) (layer F.Cu) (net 6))
 (segment (start 127.555981 65.813337) (end 130.631347 62.737973) (width 1) (layer F.Cu) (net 6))
 (segment (start 130.631347 62.737973) (end 137.879977 62.737973) (width 1) (layer F.Cu) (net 6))
 (segment (start 137.879977 62.737973) (end 151.815999 76.673995) (width 1) (layer F.Cu) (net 6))
 (segment (start 153.924 89.408) (end 153.416006 89.408) (width 1) (layer B.Cu) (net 6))
 (segment (start 172.212 89.408) (end 153.924 89.408) (width 1) (layer B.Cu) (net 6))
 (segment (start 132.588 86.868) (end 131.385919 86.868) (width 1) (layer F.Cu) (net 7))
 (segment (start 150.783997 72.552005) (end 151.383996 73.152004) (width 1) (layer F.Cu) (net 7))
 (segment (start 130.010023 61.237962) (end 139.469954 61.237962) (width 1) (layer F.Cu) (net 7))
 (segment (start 131.385919 86.868) (end 125.984 81.466081) (width 1) (layer F.Cu) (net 7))
 (segment (start 139.469954 61.237962) (end 150.783997 72.552005) (width 1) (layer F.Cu) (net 7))
 (segment (start 125.984 65.263983) (end 130.010023 61.237962) (width 1) (layer F.Cu) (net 7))
 (segment (start 125.984 81.466081) (end 125.984 65.263983) (width 1) (layer F.Cu) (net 7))
 (via (at 151.383996 73.152004) (size 1.2) (drill 0.7) (layers F.Cu B.Cu) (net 7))
 (segment (start 151.983995 73.752003) (end 151.383996 73.152004) (width 1) (layer B.Cu) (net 7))
 (segment (start 172.212 75.692) (end 153.923992 75.692) (width 1) (layer B.Cu) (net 7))
 (segment (start 153.923992 75.692) (end 151.983995 73.752003) (width 1) (layer B.Cu) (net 7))
 (segment (start 143.763992 86.868) (end 143.764 86.868008) (width 1) (layer F.Cu) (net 8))
 (segment (start 135.128 86.868) (end 143.763992 86.868) (width 1) (layer F.Cu) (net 8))
 (via (at 143.764 86.868008) (size 1.2) (drill 0.7) (layers F.Cu B.Cu) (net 8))
 (segment (start 143.764 87.716536) (end 143.764 86.868008) (width 1) (layer B.Cu) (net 8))
 (segment (start 143.764 92.964) (end 143.764 87.716536) (width 1) (layer B.Cu) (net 8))
 (segment (start 172.212 94.488) (end 145.288 94.488) (width 1) (layer B.Cu) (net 8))
 (segment (start 145.288 94.488) (end 143.764 92.964) (width 1) (layer B.Cu) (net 8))
 (via (at 145.461793 89.408) (size 1.2) (drill 0.7) (layers F.Cu B.Cu) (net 9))
 (segment (start 135.128 89.408) (end 145.461793 89.408) (width 1) (layer F.Cu) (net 9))
 (segment (start 146.061792 88.808001) (end 145.461793 89.408) (width 1) (layer B.Cu) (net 9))
 (segment (start 172.212 86.868) (end 148.001793 86.868) (width 1) (layer B.Cu) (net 9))
 (segment (start 148.001793 86.868) (end 146.061792 88.808001) (width 1) (layer B.Cu) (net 9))
 (segment (start 132.588 94.488) (end 131.385919 94.488) (width 1) (layer F.Cu) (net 10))
 (via (at 153.416 78.232) (size 1.2) (drill 0.7) (layers F.Cu B.Cu) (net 10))
 (segment (start 153.416 77.383472) (end 153.416 78.232) (width 1) (layer F.Cu) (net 10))
 (segment (start 129.388699 59.737955) (end 140.533623 59.737955) (width 1) (layer F.Cu) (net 10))
 (segment (start 153.416 72.620332) (end 153.416 77.383472) (width 1) (layer F.Cu) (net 10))
 (segment (start 128.586279 60.540371) (end 129.388699 59.737955) (width 1) (layer F.Cu) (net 10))
 (segment (start 124.483991 87.586072) (end 124.483991 64.642657) (width 1) (layer F.Cu) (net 10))
 (segment (start 140.533623 59.737955) (end 153.416 72.620332) (width 1) (layer F.Cu) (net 10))
 (segment (start 124.483991 64.642657) (end 128.586279 60.540371) (width 1) (layer F.Cu) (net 10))
 (segment (start 131.385919 94.488) (end 124.483991 87.586072) (width 1) (layer F.Cu) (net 10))
 (segment (start 172.212 78.232) (end 153.416 78.232) (width 1) (layer B.Cu) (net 10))
 (via (at 153.416 69.596026) (size 1.2) (drill 0.7) (layers F.Cu B.Cu) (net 11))
 (segment (start 152.567472 69.596026) (end 153.416 69.596026) (width 1) (layer F.Cu) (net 11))
 (segment (start 141.20939 58.237944) (end 152.567472 69.596026) (width 1) (layer F.Cu) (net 11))
 (segment (start 132.588 97.028) (end 131.385919 97.028) (width 1) (layer F.Cu) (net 11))
 (segment (start 122.98398 88.626061) (end 122.98398 64.021312) (width 1) (layer F.Cu) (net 11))
 (segment (start 131.385919 97.028) (end 122.98398 88.626061) (width 1) (layer F.Cu) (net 11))
 (segment (start 122.98398 64.021312) (end 128.767377 58.237944) (width 1) (layer F.Cu) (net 11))
 (segment (start 128.767377 58.237944) (end 141.20939 58.237944) (width 1) (layer F.Cu) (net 11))
 (segment (start 154.015999 70.196025) (end 153.416 69.596026) (width 1) (layer B.Cu) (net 11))
 (segment (start 172.212 73.152) (end 156.971974 73.152) (width 1) (layer B.Cu) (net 11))
 (segment (start 156.971974 73.152) (end 154.015999 70.196025) (width 1) (layer B.Cu) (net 11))
 (via (at 143.764 57.912) (size 1.2) (drill 0.7) (layers F.Cu B.Cu) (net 12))
 (segment (start 121.48391 63.400046) (end 128.146054 56.737935) (width 1) (layer F.Cu) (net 12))
 (segment (start 121.48391 94.745991) (end 121.48391 63.400046) (width 1) (layer F.Cu) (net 12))
 (segment (start 142.589935 56.737935) (end 143.164001 57.312001) (width 1) (layer F.Cu) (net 12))
 (segment (start 128.146054 56.737935) (end 142.589935 56.737935) (width 1) (layer F.Cu) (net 12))
 (segment (start 143.164001 57.312001) (end 143.764 57.912) (width 1) (layer F.Cu) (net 12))
 (segment (start 131.385919 104.648) (end 121.48391 94.745991) (width 1) (layer F.Cu) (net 12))
 (segment (start 132.588 104.648) (end 131.385919 104.648) (width 1) (layer F.Cu) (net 12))
 (segment (start 145.796 55.88) (end 144.363999 57.312001) (width 1) (layer B.Cu) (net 12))
 (segment (start 144.363999 57.312001) (end 143.764 57.912) (width 1) (layer B.Cu) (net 12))
 (segment (start 159.512 55.88) (end 145.796 55.88) (width 1) (layer B.Cu) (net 12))
 (segment (start 144.645922 55.237924) (end 148.244 58.836002) (width 1) (layer F.Cu) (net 13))
 (segment (start 119.983902 95.785983) (end 119.983902 62.778717) (width 1) (layer F.Cu) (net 13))
 (segment (start 132.588 107.188) (end 131.385919 107.188) (width 1) (layer F.Cu) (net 13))
 (segment (start 148.244 58.836002) (end 148.843999 59.436001) (width 1) (layer F.Cu) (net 13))
 (segment (start 119.983902 62.778717) (end 127.524732 55.237924) (width 1) (layer F.Cu) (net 13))
 (segment (start 131.385919 107.188) (end 119.983902 95.785983) (width 1) (layer F.Cu) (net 13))
 (segment (start 127.524732 55.237924) (end 144.645922 55.237924) (width 1) (layer F.Cu) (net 13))
 (via (at 148.843999 59.436001) (size 1.2) (drill 0.7) (layers F.Cu B.Cu) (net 13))
 (segment (start 162.052 55.88) (end 162.052 57.912) (width 1) (layer B.Cu) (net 13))
 (segment (start 149.692527 59.436001) (end 148.843999 59.436001) (width 1) (layer B.Cu) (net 13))
 (segment (start 160.528 59.436) (end 149.692527 59.436001) (width 1) (layer B.Cu) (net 13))
 (segment (start 162.052 57.912) (end 160.528 59.436) (width 1) (layer B.Cu) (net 13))
 (segment (start 135.128 107.188) (end 143.764 107.188) (width 1) (layer F.Cu) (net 14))
 (via (at 143.764 107.188) (size 1.2) (drill 0.7) (layers F.Cu B.Cu) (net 14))
 (segment (start 141.563999 104.987999) (end 143.164001 106.588001) (width 1) (layer B.Cu) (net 14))
 (segment (start 167.276042 65.895958) (end 149.914708 65.895958) (width 1) (layer B.Cu) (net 14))
 (segment (start 169.164 64.008) (end 167.276042 65.895958) (width 1) (layer B.Cu) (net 14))
 (segment (start 149.914708 65.895958) (end 143.764 72.046666) (width 1) (layer B.Cu) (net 14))
 (segment (start 143.764 72.046666) (end 143.764 81.28) (width 1) (layer B.Cu) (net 14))
 (segment (start 143.164001 106.588001) (end 143.764 107.188) (width 1) (layer B.Cu) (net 14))
 (segment (start 143.764 81.28) (end 141.563999 83.480001) (width 1) (layer B.Cu) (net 14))
 (segment (start 141.563999 83.480001) (end 141.563999 104.987999) (width 1) (layer B.Cu) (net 14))
 (segment (start 169.672 63.5) (end 169.672 55.88) (width 1) (layer B.Cu) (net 14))
 (segment (start 169.164 64.008) (end 169.672 63.5) (width 1) (layer B.Cu) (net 14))
 (via (at 153.416 61.468028) (size 1.2) (drill 0.7) (layers F.Cu B.Cu) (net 15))
 (segment (start 153.416 59.01175) (end 153.416 61.468028) (width 1) (layer F.Cu) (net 15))
 (segment (start 131.385919 109.728) (end 118.364 96.706081) (width 1) (layer F.Cu) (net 15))
 (segment (start 132.588 109.728) (end 131.385919 109.728) (width 1) (layer F.Cu) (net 15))
 (segment (start 118.364 96.706081) (end 118.364 61.976) (width 1) (layer F.Cu) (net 15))
 (segment (start 118.364 61.976) (end 126.602082 53.737918) (width 1) (layer F.Cu) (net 15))
 (segment (start 126.602082 53.737918) (end 148.142168 53.737918) (width 1) (layer F.Cu) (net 15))
 (segment (start 148.142168 53.737918) (end 153.416 59.01175) (width 1) (layer F.Cu) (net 15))
 (segment (start 164.592 59.944) (end 164.592 55.88) (width 1) (layer B.Cu) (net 15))
 (segment (start 153.416 61.468028) (end 163.067972 61.468028) (width 1) (layer B.Cu) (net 15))
 (segment (start 163.067972 61.468028) (end 164.592 59.944) (width 1) (layer B.Cu) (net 15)))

